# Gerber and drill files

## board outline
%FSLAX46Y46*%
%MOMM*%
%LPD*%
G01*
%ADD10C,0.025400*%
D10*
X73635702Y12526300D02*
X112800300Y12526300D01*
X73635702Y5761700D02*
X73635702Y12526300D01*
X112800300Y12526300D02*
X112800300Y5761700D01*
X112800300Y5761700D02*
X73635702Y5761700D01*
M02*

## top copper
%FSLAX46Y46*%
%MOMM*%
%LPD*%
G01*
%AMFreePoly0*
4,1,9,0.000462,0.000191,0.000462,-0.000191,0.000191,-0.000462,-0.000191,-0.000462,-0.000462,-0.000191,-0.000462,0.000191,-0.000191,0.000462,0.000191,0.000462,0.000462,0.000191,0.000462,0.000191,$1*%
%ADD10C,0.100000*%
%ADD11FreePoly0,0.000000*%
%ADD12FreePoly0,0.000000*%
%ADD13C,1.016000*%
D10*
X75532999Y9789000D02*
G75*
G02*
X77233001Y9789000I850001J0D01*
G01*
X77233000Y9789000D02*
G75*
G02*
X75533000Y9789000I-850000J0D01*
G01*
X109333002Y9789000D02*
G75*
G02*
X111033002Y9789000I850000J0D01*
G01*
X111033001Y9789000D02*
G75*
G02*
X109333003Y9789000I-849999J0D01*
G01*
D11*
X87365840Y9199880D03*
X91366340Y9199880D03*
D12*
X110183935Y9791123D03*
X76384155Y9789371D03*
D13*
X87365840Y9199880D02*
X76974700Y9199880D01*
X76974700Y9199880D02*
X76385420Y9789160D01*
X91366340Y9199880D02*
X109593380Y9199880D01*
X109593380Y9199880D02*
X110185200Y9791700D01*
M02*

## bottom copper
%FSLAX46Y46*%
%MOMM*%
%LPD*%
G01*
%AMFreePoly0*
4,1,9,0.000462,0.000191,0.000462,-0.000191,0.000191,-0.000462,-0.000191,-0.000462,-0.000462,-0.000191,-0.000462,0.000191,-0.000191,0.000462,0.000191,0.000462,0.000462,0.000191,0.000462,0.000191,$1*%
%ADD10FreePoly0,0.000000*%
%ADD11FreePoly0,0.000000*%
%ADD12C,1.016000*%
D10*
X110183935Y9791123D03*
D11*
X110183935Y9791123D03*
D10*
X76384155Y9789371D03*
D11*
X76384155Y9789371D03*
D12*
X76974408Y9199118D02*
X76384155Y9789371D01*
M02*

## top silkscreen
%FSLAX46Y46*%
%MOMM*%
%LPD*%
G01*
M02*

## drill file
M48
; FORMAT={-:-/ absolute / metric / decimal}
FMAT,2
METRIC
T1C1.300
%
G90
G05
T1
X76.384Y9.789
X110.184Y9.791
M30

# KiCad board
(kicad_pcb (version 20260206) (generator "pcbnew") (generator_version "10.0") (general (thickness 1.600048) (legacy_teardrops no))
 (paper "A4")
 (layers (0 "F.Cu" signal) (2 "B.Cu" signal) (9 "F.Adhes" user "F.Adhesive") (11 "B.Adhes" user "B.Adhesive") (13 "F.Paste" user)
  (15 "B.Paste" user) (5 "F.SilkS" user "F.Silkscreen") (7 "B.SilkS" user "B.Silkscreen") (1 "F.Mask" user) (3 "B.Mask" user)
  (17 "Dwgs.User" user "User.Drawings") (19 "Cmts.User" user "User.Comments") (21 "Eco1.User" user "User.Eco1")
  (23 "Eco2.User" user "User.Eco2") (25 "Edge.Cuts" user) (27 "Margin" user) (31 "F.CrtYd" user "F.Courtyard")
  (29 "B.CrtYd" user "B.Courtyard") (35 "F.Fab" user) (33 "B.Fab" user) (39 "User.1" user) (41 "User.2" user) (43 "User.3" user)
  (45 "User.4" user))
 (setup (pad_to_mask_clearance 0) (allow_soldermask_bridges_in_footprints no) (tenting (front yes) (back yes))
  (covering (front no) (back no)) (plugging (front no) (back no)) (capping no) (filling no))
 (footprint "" (layer "F.Cu") (at 0 0)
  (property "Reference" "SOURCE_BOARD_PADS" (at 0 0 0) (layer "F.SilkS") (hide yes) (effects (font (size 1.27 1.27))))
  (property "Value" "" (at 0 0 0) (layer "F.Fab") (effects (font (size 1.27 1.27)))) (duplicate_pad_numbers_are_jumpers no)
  (pad "1" smd custom (at 87.36584 -9.19988) (size 0.001 0.001) (layers "F.Cu" "F.Mask" "F.Paste") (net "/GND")
   (options (clearance outline) (anchor circle)) (primitives))
  (pad "2" smd custom (at 91.36634 -9.19988) (size 0.001 0.001) (layers "F.Cu" "F.Mask" "F.Paste") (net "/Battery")
   (options (clearance outline) (anchor circle)) (primitives)))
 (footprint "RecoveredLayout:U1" (layer "B.Cu") (at 110.183935 -9.791123)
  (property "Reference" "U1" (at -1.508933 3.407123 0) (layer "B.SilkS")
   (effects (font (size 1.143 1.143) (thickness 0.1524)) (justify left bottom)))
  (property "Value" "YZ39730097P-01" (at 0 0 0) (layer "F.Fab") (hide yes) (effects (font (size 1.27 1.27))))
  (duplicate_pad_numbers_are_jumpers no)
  (pad "1" thru_hole custom (at 0 0) (size 0.001 0.001) (drill 1.300023) (layers "*.Cu") (remove_unused_layers no) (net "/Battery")
   (options (clearance outline) (anchor circle)) (primitives))
  (pad "1" smd custom (at 0 0) (size 0.001 0.001) (layers "B.Cu" "B.Mask" "B.Paste") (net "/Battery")
   (options (clearance outline) (anchor circle)) (primitives)))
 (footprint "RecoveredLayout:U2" (layer "B.Cu") (at 76.384155 -9.789371)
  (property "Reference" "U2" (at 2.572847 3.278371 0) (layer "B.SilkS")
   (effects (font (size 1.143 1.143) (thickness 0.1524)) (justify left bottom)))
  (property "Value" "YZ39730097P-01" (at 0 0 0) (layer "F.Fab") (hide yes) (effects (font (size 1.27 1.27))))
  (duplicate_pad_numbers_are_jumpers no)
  (pad "1" thru_hole custom (at 0 0) (size 0.001 0.001) (drill 1.300023) (layers "*.Cu") (remove_unused_layers no) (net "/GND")
   (options (clearance outline) (anchor circle)) (primitives))
  (pad "1" smd custom (at 0 0) (size 0.001 0.001) (layers "B.Cu" "B.Mask" "B.Paste") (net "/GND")
   (options (clearance outline) (anchor circle)) (primitives)))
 (gr_arc (start 75.532999 -9.789) (mid 76.401288 -10.638804) (end 77.233 -9.789) (stroke (width 0.1) (type default)) (layer "F.Cu")
  (net "/GND"))
 (gr_arc (start 77.233 -9.789) (mid 76.364711 -8.939196) (end 75.532999 -9.789) (stroke (width 0.1) (type default)) (layer "F.Cu")
  (net "/GND"))
 (gr_arc (start 109.333002 -9.789) (mid 110.20129 -10.638803) (end 111.033001 -9.789) (stroke (width 0.1) (type default)) (layer "F.Cu")
  (net "/Battery"))
 (gr_arc (start 111.033001 -9.789) (mid 110.164713 -8.939197) (end 109.333002 -9.789) (stroke (width 0.1) (type default)) (layer "F.Cu")
  (net "/Battery"))
 (gr_line (start 73.635702 -12.5263) (end 112.8003 -12.5263) (stroke (width 0.0254) (type default)) (layer "Edge.Cuts"))
 (gr_line (start 73.635702 -5.7617) (end 73.635702 -12.5263) (stroke (width 0.0254) (type default)) (layer "Edge.Cuts"))
 (gr_line (start 112.8003 -12.5263) (end 112.8003 -5.7617) (stroke (width 0.0254) (type default)) (layer "Edge.Cuts"))
 (gr_line (start 112.8003 -5.7617) (end 73.635702 -5.7617) (stroke (width 0.0254) (type default)) (layer "Edge.Cuts"))
 (segment (start 87.36584 -9.19988) (end 76.9747 -9.19988) (width 1.016) (layer "F.Cu") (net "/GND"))
 (segment (start 76.9747 -9.19988) (end 76.38542 -9.78916) (width 1.016) (layer "F.Cu") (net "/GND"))
 (segment (start 76.974408 -9.199118) (end 76.384155 -9.789371) (width 1.016) (layer "B.Cu") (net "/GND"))
 (segment (start 91.36634 -9.19988) (end 109.59338 -9.19988) (width 1.016) (layer "F.Cu") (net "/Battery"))
 (segment (start 109.59338 -9.19988) (end 110.1852 -9.7917) (width 1.016) (layer "F.Cu") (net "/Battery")))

